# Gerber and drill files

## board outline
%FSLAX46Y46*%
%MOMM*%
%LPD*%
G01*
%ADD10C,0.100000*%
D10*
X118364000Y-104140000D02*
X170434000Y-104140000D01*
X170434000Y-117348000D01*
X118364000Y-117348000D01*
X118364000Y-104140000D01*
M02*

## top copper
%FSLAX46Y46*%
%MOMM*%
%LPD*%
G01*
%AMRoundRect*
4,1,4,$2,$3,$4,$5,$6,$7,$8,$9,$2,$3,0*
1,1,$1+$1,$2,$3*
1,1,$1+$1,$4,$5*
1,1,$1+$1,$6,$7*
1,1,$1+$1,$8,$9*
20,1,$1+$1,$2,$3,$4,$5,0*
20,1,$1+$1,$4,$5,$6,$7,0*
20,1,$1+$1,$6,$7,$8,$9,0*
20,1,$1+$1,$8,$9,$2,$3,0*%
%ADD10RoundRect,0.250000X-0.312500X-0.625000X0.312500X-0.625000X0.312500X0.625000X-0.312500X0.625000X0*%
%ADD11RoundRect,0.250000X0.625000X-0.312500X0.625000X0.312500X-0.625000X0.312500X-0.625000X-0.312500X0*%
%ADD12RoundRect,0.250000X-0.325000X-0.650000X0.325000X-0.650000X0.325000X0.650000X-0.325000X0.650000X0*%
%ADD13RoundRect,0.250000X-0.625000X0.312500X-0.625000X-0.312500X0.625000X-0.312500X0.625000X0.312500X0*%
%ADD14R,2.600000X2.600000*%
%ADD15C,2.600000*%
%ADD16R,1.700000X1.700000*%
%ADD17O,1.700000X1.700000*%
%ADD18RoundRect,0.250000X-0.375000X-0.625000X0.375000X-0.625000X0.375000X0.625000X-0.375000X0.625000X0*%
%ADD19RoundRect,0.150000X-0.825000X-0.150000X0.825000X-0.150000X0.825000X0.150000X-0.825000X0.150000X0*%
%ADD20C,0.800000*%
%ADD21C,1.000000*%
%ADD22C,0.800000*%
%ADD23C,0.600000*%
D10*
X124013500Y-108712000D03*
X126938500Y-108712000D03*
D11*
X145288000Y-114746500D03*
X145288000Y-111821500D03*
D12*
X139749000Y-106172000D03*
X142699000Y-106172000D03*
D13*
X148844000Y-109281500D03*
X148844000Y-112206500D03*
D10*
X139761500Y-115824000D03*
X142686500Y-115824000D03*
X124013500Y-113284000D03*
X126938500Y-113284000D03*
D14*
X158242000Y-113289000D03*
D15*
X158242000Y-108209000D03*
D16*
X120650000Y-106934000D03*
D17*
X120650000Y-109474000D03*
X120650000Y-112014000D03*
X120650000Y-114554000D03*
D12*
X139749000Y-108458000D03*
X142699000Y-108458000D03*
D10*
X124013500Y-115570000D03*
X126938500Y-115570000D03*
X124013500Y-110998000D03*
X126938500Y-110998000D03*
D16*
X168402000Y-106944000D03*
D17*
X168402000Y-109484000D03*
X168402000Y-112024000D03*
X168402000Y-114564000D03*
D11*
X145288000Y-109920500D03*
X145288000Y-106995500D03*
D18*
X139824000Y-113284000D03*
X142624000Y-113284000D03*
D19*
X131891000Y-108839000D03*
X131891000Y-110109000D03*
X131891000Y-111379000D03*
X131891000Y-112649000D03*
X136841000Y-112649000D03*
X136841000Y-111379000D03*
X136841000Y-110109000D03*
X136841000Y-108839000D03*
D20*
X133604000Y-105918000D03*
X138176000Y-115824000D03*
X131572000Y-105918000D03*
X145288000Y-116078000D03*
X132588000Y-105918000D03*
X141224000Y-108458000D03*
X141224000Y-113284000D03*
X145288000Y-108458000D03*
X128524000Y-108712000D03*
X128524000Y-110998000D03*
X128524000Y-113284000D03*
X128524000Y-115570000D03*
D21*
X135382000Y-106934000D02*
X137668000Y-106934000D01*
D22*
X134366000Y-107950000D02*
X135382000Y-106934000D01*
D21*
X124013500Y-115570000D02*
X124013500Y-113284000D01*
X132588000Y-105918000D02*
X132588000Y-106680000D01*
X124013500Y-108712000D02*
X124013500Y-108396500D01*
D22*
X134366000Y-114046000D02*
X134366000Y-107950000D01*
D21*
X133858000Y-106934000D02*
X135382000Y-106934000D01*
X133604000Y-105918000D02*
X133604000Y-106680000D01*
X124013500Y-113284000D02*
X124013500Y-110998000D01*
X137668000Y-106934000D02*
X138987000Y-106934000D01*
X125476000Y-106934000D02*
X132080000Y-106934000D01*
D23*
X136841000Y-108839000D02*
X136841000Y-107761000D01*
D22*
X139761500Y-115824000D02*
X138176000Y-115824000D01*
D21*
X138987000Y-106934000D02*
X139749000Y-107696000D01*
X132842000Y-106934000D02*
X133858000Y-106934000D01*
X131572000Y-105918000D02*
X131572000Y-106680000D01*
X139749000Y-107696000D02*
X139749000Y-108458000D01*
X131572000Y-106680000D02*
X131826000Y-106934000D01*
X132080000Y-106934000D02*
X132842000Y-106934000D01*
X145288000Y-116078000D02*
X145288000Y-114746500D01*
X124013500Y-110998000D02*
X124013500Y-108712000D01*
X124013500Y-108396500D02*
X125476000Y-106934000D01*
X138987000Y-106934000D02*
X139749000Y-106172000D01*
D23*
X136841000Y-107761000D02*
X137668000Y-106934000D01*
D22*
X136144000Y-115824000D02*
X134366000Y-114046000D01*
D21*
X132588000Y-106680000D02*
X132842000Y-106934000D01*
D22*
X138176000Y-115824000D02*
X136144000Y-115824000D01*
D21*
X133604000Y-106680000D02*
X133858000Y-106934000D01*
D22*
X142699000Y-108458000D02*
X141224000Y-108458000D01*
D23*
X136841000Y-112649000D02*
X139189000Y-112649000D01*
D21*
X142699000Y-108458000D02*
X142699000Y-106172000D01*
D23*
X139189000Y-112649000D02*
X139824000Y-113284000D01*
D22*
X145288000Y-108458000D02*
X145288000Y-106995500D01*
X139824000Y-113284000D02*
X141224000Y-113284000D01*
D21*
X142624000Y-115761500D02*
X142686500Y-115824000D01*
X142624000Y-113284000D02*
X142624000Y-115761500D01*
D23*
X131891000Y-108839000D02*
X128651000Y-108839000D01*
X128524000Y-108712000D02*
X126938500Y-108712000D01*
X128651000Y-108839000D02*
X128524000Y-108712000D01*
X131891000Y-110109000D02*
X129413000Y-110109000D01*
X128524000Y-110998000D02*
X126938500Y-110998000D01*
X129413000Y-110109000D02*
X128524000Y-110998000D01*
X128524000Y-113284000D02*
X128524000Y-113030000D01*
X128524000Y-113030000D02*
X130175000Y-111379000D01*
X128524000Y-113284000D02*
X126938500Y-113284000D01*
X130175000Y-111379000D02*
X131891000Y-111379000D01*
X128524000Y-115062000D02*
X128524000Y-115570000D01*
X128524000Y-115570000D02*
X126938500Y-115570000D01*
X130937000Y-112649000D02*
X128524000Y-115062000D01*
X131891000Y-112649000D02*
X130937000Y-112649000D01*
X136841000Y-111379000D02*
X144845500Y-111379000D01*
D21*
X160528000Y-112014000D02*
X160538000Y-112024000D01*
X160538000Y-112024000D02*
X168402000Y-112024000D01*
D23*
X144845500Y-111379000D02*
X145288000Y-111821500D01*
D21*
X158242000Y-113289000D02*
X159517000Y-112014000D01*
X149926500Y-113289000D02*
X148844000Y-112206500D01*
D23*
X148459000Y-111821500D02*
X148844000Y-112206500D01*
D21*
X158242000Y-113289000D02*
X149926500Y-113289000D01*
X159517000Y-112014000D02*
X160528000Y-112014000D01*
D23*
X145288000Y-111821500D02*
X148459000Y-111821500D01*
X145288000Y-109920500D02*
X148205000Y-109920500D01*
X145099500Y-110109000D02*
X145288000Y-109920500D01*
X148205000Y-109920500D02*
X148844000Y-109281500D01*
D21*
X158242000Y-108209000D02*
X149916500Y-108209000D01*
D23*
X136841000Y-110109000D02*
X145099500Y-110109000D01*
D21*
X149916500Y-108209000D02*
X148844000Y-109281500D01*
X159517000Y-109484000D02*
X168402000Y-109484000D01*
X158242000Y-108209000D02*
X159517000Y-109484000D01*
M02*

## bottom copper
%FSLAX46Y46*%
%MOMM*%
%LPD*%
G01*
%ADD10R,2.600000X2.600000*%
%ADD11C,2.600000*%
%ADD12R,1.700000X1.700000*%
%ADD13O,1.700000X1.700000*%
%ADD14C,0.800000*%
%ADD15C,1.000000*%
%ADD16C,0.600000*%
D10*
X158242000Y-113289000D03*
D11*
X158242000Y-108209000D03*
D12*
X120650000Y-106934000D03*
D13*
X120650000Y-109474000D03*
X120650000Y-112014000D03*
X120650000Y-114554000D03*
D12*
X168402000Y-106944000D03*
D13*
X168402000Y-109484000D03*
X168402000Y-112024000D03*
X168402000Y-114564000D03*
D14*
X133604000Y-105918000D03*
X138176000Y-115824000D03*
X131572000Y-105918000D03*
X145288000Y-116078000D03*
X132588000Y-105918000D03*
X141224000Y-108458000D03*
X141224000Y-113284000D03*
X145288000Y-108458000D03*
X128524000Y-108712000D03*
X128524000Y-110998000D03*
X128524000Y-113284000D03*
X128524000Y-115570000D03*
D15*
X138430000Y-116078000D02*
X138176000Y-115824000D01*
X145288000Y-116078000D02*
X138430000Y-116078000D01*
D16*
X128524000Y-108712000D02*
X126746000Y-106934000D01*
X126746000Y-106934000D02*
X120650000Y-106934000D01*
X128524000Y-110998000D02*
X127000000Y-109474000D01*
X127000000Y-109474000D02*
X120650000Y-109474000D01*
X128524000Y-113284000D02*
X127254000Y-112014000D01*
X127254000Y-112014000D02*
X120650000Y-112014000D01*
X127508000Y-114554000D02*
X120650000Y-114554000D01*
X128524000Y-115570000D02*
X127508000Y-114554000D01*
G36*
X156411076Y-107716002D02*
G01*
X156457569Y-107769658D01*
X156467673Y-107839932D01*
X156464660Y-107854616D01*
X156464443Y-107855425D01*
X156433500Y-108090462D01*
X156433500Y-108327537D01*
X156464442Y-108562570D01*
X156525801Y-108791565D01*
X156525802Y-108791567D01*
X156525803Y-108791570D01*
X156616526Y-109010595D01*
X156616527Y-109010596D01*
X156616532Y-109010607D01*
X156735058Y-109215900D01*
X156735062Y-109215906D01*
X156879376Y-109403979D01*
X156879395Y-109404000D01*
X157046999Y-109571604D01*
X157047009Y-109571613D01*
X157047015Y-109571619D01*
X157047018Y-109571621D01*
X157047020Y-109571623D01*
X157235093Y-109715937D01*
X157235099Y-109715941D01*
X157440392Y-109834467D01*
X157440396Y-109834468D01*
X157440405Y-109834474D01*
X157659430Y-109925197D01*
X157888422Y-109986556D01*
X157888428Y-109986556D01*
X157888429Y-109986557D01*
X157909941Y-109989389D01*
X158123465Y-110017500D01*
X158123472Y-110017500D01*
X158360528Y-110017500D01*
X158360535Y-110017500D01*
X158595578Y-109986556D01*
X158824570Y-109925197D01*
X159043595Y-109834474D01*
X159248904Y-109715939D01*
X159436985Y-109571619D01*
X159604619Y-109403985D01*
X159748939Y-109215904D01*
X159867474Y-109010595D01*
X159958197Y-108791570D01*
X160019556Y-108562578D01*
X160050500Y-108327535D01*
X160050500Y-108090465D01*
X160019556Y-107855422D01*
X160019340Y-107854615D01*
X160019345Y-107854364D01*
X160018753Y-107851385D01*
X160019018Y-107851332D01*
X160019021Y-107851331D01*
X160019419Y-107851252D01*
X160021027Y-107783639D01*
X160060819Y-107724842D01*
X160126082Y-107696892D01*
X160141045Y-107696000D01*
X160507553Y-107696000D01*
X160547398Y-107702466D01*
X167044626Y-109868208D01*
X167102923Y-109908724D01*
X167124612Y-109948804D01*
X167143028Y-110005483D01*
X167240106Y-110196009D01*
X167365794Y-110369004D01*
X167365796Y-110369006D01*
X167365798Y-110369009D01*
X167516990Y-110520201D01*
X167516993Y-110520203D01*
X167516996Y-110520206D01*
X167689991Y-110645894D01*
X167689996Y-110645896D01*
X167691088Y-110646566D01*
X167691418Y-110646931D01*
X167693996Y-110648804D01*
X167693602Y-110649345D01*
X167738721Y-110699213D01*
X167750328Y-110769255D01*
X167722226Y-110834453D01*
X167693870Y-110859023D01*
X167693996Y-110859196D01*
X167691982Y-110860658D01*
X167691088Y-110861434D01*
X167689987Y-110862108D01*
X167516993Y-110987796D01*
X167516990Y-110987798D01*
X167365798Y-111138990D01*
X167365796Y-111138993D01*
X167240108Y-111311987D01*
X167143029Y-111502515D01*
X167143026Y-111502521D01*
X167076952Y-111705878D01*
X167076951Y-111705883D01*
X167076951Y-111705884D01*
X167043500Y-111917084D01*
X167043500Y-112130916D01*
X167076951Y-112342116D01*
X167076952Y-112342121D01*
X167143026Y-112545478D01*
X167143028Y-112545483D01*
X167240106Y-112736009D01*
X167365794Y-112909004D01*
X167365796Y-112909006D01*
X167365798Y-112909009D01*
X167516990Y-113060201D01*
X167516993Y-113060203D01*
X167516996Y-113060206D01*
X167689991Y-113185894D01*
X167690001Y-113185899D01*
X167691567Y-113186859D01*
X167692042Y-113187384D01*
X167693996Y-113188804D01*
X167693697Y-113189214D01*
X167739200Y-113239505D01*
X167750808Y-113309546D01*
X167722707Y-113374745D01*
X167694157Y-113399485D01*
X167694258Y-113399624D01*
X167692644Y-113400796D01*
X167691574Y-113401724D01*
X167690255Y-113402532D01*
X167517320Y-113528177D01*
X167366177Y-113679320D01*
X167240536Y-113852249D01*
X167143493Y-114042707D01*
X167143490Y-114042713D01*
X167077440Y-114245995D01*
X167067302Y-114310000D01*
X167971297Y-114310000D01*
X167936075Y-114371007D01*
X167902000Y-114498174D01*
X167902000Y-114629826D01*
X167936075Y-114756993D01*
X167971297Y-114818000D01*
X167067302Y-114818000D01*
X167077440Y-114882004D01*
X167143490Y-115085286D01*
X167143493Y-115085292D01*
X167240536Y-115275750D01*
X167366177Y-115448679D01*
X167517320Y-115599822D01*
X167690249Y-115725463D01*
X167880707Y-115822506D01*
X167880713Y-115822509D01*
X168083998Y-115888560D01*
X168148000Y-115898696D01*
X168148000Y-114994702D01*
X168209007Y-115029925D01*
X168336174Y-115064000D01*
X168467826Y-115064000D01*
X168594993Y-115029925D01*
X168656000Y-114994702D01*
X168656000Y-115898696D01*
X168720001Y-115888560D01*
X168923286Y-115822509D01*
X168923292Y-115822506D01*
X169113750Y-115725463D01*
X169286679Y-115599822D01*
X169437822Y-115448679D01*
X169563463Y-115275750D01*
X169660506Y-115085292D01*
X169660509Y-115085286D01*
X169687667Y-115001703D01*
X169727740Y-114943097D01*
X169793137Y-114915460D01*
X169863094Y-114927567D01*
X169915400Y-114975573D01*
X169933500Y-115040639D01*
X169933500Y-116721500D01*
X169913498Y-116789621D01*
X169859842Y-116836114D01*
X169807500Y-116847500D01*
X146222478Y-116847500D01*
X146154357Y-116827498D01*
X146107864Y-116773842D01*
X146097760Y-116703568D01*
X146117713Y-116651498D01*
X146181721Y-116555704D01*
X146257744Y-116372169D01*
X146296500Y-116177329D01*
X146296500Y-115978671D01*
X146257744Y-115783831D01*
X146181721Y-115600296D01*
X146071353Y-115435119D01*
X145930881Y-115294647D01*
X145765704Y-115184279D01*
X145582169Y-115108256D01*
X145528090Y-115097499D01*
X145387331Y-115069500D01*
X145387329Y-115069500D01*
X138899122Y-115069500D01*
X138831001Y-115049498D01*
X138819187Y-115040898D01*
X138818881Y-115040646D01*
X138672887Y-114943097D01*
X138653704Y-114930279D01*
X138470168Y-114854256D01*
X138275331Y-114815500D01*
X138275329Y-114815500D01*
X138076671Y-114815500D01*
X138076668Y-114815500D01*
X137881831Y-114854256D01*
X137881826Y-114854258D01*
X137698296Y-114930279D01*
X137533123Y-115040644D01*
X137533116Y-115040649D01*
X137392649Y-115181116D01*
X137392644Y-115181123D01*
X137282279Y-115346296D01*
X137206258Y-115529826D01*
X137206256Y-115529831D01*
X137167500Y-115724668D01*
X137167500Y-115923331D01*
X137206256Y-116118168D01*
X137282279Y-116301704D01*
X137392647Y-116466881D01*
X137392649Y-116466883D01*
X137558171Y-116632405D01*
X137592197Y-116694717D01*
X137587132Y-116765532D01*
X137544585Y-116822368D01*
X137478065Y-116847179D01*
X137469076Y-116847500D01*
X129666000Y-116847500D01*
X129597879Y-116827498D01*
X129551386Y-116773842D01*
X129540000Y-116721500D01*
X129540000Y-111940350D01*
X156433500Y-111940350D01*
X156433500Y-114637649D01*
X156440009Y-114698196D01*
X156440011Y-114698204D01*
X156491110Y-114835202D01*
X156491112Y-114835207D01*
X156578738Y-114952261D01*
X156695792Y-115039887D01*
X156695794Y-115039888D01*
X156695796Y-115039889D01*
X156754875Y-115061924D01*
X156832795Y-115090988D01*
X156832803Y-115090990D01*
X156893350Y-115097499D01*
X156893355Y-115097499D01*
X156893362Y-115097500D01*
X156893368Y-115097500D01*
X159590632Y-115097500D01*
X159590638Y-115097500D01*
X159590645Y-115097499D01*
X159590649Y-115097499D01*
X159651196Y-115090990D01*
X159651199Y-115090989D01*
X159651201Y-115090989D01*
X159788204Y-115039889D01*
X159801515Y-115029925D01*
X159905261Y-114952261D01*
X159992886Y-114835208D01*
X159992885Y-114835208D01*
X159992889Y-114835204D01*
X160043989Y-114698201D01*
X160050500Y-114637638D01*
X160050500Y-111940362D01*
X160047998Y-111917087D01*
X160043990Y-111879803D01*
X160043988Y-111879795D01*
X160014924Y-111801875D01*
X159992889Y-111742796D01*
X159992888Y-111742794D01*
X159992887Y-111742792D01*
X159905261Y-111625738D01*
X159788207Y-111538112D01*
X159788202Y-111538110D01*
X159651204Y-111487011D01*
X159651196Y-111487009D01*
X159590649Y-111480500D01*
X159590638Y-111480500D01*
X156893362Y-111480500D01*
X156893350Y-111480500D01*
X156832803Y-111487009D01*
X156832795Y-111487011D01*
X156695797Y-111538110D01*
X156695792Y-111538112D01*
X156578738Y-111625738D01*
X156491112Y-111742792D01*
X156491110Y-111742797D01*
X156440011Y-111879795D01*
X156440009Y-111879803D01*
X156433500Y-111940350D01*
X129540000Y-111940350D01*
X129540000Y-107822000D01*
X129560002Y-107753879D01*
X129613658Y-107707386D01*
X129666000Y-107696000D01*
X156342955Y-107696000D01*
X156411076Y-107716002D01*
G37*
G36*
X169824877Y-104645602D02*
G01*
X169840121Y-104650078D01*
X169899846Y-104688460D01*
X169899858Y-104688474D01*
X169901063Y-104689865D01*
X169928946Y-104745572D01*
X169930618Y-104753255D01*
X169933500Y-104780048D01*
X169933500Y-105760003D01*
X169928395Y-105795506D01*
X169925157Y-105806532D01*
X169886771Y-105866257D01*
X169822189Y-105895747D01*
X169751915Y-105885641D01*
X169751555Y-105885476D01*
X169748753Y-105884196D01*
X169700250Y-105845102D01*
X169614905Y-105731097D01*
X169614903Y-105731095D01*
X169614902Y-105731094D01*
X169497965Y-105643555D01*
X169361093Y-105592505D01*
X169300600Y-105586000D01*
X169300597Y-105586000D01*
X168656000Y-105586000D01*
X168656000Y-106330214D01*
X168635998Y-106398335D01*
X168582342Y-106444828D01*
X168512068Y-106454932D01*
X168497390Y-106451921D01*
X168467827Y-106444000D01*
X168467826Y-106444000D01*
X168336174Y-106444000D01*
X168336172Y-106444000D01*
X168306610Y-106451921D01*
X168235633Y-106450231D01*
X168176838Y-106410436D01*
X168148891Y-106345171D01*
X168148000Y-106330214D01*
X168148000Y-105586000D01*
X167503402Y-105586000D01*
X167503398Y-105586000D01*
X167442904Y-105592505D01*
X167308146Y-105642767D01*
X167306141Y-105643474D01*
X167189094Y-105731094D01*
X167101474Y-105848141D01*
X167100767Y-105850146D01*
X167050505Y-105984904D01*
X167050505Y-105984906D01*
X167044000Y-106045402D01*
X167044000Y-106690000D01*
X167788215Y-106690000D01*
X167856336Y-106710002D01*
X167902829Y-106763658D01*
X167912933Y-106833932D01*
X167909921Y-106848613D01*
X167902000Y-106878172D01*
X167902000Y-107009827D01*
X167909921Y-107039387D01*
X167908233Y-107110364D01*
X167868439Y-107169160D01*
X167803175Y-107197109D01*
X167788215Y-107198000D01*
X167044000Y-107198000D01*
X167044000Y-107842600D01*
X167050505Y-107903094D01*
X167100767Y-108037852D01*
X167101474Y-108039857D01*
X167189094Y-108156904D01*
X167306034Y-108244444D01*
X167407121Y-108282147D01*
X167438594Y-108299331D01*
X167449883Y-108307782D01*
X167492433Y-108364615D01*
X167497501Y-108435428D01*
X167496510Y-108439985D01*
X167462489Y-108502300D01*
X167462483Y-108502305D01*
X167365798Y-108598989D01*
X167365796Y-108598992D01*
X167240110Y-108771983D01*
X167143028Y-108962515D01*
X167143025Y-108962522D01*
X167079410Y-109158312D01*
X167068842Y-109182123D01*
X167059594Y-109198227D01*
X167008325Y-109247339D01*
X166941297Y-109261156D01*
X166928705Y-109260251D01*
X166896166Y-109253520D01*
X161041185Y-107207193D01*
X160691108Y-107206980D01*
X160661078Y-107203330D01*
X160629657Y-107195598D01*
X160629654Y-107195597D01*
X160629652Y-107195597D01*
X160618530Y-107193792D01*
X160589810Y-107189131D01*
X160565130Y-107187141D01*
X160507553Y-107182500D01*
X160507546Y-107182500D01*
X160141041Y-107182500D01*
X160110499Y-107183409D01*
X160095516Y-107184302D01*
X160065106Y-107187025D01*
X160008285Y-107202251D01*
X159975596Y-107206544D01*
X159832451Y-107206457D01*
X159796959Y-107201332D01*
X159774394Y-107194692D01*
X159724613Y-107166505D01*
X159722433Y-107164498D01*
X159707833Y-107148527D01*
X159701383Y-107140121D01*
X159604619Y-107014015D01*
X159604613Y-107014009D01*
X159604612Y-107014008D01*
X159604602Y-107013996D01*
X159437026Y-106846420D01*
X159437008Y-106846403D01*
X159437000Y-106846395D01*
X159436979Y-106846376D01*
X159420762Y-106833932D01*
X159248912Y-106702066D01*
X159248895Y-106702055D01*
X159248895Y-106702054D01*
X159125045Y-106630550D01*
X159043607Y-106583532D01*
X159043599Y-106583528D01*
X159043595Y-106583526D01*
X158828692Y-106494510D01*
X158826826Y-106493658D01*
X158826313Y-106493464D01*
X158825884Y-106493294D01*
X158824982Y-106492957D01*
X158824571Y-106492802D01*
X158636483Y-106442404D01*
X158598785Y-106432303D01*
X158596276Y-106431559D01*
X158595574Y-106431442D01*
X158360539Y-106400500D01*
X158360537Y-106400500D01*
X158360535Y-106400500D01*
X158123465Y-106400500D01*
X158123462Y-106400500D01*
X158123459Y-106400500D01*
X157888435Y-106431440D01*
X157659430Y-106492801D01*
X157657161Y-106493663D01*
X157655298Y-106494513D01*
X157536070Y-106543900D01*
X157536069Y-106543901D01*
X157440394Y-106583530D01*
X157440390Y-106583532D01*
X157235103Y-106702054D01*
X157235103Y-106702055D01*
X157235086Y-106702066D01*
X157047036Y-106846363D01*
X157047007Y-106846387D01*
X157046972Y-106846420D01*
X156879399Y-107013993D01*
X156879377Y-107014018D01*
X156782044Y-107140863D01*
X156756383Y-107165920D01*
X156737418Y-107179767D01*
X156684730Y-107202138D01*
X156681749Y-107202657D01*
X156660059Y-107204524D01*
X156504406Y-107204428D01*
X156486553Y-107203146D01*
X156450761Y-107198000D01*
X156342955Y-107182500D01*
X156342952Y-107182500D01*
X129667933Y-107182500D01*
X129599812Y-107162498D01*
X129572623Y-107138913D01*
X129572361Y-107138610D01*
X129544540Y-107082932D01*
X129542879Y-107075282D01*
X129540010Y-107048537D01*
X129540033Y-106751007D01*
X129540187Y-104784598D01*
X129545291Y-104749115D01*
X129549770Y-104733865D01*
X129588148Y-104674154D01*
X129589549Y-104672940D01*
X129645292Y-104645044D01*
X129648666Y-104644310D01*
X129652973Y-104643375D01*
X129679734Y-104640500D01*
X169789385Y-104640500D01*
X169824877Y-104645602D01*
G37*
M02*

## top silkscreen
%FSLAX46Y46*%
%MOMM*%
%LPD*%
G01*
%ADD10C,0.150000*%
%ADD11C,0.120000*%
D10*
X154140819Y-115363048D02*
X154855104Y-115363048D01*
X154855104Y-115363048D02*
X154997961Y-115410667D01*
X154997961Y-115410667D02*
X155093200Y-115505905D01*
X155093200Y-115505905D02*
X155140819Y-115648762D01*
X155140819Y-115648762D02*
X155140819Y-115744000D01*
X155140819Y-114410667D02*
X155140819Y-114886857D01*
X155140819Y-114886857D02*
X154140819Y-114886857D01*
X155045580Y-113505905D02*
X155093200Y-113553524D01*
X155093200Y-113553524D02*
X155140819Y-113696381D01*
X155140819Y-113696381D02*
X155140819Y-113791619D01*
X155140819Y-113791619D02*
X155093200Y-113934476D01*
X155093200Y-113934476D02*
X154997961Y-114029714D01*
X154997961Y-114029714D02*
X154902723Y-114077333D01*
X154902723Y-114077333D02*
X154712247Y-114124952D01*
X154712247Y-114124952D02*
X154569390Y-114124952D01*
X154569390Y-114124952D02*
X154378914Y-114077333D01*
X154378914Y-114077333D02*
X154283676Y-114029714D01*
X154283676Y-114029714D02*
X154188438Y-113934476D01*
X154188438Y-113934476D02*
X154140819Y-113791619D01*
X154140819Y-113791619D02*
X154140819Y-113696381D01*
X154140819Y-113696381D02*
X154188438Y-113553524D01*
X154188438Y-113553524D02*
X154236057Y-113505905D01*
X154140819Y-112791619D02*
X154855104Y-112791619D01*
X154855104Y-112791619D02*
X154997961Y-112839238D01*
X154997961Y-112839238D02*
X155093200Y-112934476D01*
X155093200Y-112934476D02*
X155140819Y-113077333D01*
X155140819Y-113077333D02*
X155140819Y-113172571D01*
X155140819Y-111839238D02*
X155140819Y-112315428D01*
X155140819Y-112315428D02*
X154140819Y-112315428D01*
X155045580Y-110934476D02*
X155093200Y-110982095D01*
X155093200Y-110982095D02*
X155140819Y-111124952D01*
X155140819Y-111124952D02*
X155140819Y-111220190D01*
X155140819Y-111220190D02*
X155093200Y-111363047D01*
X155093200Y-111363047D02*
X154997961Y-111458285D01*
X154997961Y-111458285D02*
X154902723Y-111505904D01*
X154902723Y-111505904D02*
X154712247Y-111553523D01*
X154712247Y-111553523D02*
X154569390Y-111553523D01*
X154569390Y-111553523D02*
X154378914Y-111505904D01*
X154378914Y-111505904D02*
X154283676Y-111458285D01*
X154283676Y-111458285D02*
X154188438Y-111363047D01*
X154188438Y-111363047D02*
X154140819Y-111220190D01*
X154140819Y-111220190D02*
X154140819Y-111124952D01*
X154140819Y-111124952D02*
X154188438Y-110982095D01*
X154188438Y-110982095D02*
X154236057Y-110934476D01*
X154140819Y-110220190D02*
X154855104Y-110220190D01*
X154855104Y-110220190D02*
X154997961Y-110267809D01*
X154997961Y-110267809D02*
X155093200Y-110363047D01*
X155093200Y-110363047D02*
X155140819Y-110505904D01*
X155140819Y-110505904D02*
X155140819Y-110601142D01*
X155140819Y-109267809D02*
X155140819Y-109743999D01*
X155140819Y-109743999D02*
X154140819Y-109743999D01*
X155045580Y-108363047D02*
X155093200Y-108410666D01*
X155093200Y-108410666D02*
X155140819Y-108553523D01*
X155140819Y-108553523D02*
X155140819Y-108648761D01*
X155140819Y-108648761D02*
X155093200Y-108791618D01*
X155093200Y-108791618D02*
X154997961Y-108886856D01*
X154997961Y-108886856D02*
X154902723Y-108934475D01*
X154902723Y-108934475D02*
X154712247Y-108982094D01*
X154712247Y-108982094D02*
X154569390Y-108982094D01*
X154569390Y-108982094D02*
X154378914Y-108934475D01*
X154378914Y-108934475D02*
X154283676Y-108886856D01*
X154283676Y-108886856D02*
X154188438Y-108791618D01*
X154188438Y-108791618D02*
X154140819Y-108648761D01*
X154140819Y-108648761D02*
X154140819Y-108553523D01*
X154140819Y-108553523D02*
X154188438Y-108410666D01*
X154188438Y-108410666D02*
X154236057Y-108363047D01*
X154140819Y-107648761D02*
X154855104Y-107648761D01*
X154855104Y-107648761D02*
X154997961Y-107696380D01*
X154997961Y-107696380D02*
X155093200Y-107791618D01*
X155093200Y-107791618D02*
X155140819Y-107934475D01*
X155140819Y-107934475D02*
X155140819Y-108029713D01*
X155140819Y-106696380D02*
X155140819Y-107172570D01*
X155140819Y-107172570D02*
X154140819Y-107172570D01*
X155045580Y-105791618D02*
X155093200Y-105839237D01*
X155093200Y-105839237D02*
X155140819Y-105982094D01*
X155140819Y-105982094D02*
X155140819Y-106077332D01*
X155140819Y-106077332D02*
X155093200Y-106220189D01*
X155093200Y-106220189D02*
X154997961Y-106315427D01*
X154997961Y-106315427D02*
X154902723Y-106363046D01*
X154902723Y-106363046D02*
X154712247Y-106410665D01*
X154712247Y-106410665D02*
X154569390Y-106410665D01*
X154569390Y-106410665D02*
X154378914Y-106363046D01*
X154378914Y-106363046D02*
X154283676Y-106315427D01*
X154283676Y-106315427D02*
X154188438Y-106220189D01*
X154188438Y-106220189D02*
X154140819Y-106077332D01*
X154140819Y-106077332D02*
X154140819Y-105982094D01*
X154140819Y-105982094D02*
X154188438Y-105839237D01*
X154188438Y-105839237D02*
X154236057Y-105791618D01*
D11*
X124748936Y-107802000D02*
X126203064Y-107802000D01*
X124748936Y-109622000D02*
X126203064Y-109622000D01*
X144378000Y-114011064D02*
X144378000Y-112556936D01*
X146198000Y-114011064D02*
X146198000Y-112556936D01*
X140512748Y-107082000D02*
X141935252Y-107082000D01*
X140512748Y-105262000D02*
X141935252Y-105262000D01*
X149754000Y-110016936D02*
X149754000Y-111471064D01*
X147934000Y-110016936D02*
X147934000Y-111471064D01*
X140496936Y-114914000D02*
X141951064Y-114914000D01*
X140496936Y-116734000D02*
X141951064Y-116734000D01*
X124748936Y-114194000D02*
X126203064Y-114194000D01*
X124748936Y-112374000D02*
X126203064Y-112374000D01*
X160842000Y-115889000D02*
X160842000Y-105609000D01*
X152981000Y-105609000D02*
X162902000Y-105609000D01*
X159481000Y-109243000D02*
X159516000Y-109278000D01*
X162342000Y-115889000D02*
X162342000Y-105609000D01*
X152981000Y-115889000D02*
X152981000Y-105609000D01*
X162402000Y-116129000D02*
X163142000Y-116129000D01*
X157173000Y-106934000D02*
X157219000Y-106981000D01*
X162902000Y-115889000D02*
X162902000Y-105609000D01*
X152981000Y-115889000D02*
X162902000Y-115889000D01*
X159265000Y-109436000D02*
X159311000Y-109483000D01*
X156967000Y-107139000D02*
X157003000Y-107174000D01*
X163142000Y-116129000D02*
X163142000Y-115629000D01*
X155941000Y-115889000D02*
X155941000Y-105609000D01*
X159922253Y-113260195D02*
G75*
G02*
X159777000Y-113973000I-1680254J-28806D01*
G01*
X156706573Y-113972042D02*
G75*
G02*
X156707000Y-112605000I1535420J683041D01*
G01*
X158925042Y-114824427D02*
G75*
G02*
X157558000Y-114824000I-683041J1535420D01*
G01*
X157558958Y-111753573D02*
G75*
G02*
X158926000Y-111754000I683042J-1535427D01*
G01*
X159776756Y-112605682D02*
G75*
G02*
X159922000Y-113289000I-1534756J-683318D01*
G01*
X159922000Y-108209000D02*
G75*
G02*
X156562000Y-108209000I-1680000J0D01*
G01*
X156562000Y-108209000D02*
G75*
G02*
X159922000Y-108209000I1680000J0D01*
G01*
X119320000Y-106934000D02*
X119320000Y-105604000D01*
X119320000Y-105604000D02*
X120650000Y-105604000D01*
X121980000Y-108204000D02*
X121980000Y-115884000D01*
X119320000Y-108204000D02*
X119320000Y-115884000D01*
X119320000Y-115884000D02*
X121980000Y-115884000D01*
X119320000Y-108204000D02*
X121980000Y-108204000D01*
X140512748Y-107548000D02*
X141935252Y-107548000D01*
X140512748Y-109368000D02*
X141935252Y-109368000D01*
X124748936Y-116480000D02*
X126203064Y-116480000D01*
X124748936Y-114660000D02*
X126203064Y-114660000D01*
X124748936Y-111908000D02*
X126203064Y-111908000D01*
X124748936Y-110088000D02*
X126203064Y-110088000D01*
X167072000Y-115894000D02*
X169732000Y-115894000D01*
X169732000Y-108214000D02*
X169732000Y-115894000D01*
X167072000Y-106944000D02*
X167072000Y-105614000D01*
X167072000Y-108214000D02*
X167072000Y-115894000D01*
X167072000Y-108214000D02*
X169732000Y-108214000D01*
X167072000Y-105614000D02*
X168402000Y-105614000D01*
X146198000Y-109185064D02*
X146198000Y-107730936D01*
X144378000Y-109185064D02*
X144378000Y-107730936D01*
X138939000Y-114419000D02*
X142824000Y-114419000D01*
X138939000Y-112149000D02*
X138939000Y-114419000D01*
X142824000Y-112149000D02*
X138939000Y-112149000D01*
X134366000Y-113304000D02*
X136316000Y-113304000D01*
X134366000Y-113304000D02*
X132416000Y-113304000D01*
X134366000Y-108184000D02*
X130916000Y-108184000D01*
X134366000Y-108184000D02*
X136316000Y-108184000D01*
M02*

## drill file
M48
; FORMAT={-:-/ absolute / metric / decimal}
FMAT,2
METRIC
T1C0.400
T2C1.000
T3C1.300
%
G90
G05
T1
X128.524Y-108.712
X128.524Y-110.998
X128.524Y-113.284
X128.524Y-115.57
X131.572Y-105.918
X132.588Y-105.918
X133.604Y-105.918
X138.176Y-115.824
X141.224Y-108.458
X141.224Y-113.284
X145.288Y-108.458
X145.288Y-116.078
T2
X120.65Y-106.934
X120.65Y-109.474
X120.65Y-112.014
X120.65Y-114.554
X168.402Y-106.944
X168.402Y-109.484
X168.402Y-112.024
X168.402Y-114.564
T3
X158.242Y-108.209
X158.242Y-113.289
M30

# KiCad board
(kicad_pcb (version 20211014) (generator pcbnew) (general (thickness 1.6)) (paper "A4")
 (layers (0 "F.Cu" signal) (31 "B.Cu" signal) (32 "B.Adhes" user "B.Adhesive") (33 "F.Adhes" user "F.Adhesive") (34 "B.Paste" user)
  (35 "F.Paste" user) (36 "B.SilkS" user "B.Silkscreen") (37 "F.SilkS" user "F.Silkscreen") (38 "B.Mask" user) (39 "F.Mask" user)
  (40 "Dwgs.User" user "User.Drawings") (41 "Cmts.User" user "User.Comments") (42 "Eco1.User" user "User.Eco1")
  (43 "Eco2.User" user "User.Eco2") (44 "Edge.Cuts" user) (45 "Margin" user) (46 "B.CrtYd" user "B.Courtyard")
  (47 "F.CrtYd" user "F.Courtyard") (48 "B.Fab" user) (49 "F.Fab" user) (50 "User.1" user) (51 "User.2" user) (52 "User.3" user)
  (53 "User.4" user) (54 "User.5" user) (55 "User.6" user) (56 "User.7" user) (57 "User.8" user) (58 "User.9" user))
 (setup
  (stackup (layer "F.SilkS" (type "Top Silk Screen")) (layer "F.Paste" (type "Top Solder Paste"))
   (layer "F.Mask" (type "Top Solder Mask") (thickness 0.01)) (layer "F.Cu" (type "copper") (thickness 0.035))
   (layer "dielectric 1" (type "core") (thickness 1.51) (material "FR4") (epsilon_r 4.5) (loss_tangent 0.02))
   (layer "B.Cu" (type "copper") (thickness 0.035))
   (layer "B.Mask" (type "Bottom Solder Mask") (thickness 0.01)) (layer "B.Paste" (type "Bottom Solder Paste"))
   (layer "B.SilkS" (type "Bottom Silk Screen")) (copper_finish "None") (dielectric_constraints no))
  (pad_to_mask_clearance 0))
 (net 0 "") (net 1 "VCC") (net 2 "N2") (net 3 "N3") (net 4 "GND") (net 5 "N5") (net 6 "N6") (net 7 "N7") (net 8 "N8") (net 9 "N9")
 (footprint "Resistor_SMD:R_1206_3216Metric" (layer "F.Cu") (at 125.476 108.712)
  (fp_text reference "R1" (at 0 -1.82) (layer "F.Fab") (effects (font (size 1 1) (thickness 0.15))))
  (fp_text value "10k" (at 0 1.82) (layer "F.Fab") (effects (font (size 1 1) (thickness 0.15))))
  (fp_line (start -0.727064 -0.91) (end 0.727064 -0.91) (layer "F.SilkS") (width 0.12))
  (fp_line (start -0.727064 0.91) (end 0.727064 0.91) (layer "F.SilkS") (width 0.12))
  (pad "1" smd roundrect locked (at -1.4625 0) (size 1.125 1.75) (layers "F.Cu" "F.Paste" "F.Mask") (roundrect_rratio 0.222222)
   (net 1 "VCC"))
  (pad "2" smd roundrect locked (at 1.4625 0) (size 1.125 1.75) (layers "F.Cu" "F.Paste" "F.Mask") (roundrect_rratio 0.222222) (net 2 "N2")))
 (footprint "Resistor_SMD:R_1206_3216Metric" (layer "F.Cu") (at 145.288 113.284 90)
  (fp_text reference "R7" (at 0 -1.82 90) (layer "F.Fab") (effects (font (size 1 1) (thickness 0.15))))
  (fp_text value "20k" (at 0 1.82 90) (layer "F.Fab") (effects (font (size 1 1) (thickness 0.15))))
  (fp_line (start -0.727064 -0.91) (end 0.727064 -0.91) (layer "F.SilkS") (width 0.12))
  (fp_line (start -0.727064 0.91) (end 0.727064 0.91) (layer "F.SilkS") (width 0.12))
  (pad "1" smd roundrect locked (at -1.4625 0 90) (size 1.125 1.75) (layers "F.Cu" "F.Paste" "F.Mask") (roundrect_rratio 0.222222)
   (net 1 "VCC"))
  (pad "2" smd roundrect locked (at 1.4625 0 90) (size 1.125 1.75) (layers "F.Cu" "F.Paste" "F.Mask") (roundrect_rratio 0.222222)
   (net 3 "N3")))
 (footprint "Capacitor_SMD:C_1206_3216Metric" (layer "F.Cu") (at 141.224 106.172)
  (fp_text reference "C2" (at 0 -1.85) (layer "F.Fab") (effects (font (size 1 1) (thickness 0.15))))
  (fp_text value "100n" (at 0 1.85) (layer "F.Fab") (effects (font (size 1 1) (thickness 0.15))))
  (fp_line (start -0.711252 0.91) (end 0.711252 0.91) (layer "F.SilkS") (width 0.12))
  (fp_line (start -0.711252 -0.91) (end 0.711252 -0.91) (layer "F.SilkS") (width 0.12))
  (pad "1" smd roundrect locked (at -1.475 0) (size 1.15 1.8) (layers "F.Cu" "F.Paste" "F.Mask") (roundrect_rratio 0.217391) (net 1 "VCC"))
  (pad "2" smd roundrect locked (at 1.475 0) (size 1.15 1.8) (layers "F.Cu" "F.Paste" "F.Mask") (roundrect_rratio 0.217391) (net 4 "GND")))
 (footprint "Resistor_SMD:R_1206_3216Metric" (layer "F.Cu") (at 148.844 110.744 -90)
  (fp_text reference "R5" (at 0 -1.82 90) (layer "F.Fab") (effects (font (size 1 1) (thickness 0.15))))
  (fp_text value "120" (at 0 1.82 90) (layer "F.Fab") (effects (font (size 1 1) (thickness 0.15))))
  (fp_line (start -0.727064 -0.91) (end 0.727064 -0.91) (layer "F.SilkS") (width 0.12))
  (fp_line (start -0.727064 0.91) (end 0.727064 0.91) (layer "F.SilkS") (width 0.12))
  (pad "1" smd roundrect locked (at -1.4625 0 270) (size 1.125 1.75) (layers "F.Cu" "F.Paste" "F.Mask") (roundrect_rratio 0.222222)
   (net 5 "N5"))
  (pad "2" smd roundrect locked (at 1.4625 0 270) (size 1.125 1.75) (layers "F.Cu" "F.Paste" "F.Mask") (roundrect_rratio 0.222222)
   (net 3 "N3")))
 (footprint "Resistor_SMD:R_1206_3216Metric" (layer "F.Cu") (at 141.224 115.824)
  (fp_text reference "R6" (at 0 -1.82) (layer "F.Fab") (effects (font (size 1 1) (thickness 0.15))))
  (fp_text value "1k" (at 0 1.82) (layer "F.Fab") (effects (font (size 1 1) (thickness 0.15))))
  (fp_line (start -0.727064 -0.91) (end 0.727064 -0.91) (layer "F.SilkS") (width 0.12))
  (fp_line (start -0.727064 0.91) (end 0.727064 0.91) (layer "F.SilkS") (width 0.12))
  (pad "1" smd roundrect locked (at -1.4625 0) (size 1.125 1.75) (layers "F.Cu" "F.Paste" "F.Mask") (roundrect_rratio 0.222222)
   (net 1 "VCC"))
  (pad "2" smd roundrect locked (at 1.4625 0) (size 1.125 1.75) (layers "F.Cu" "F.Paste" "F.Mask") (roundrect_rratio 0.222222) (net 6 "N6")))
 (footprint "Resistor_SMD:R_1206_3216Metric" (layer "F.Cu") (at 125.476 113.284)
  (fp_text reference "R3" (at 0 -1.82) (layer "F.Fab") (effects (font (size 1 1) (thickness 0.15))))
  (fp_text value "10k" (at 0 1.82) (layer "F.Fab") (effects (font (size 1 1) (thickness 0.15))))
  (fp_line (start -0.727064 0.91) (end 0.727064 0.91) (layer "F.SilkS") (width 0.12))
  (fp_line (start -0.727064 -0.91) (end 0.727064 -0.91) (layer "F.SilkS") (width 0.12))
  (pad "1" smd roundrect locked (at -1.4625 0) (size 1.125 1.75) (layers "F.Cu" "F.Paste" "F.Mask") (roundrect_rratio 0.222222)
   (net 1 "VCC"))
  (pad "2" smd roundrect locked (at 1.4625 0) (size 1.125 1.75) (layers "F.Cu" "F.Paste" "F.Mask") (roundrect_rratio 0.222222) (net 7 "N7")))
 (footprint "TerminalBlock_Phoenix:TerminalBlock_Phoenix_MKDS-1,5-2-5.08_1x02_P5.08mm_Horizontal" (layer "F.Cu") (at 158.242 113.289 90)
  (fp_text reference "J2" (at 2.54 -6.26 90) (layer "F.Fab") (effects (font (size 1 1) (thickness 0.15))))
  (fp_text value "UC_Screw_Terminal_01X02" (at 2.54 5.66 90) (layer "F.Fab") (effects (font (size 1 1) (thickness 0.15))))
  (fp_line (start -2.6 2.6) (end 7.68 2.6) (layer "F.SilkS") (width 0.12))
  (fp_line (start 7.68 -5.261) (end 7.68 4.66) (layer "F.SilkS") (width 0.12))
  (fp_line (start 4.046 1.239) (end 4.011 1.274) (layer "F.SilkS") (width 0.12))
  (fp_line (start -2.6 4.1) (end 7.68 4.1) (layer "F.SilkS") (width 0.12))
  (fp_line (start -2.6 -5.261) (end 7.68 -5.261) (layer "F.SilkS") (width 0.12))
  (fp_line (start -2.84 4.16) (end -2.84 4.9) (layer "F.SilkS") (width 0.12))
  (fp_line (start 6.355 -1.069) (end 6.308 -1.023) (layer "F.SilkS") (width 0.12))
  (fp_line (start -2.6 4.66) (end 7.68 4.66) (layer "F.SilkS") (width 0.12))
  (fp_line (start -2.6 -5.261) (end -2.6 4.66) (layer "F.SilkS") (width 0.12))
  (fp_line (start 3.853 1.023) (end 3.806 1.069) (layer "F.SilkS") (width 0.12))
  (fp_line (start 6.15 -1.275) (end 6.115 -1.239) (layer "F.SilkS") (width 0.12))
  (fp_line (start -2.84 4.9) (end -2.34 4.9) (layer "F.SilkS") (width 0.12))
  (fp_line (start -2.6 -2.301) (end 7.68 -2.301) (layer "F.SilkS") (width 0.12))
  (fp_arc (start 0.028805 1.680253) (mid -0.335551 1.646659) (end -0.684 1.535) (layer "F.SilkS") (width 0.12))
  (fp_arc (start -0.683042 -1.535427) (mid 0.000524 -1.680501) (end 0.684 -1.535) (layer "F.SilkS") (width 0.12))
  (fp_arc (start -1.535427 0.683042) (mid -1.680501 -0.000524) (end -1.535 -0.684) (layer "F.SilkS") (width 0.12))
  (fp_arc (start 1.535427 -0.683042) (mid 1.680501 0.000524) (end 1.535 0.684) (layer "F.SilkS") (width 0.12))
  (fp_arc (start 0.683318 1.534756) (mid 0.349292 1.643288) (end 0 1.68) (layer "F.SilkS") (width 0.12))
  (fp_circle (center 5.08 0) (end 6.76 0) (layer "F.SilkS") (width 0.12) (fill none))
  (pad "1" thru_hole rect locked (at 0 0 90) (size 2.6 2.6) (drill 1.3) (layers *.Cu *.Mask) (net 3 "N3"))
  (pad "2" thru_hole circle locked (at 5.08 0 90) (size 2.6 2.6) (drill 1.3) (layers *.Cu *.Mask) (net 5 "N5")))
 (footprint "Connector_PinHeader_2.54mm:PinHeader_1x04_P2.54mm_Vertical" (layer "F.Cu") (at 120.65 106.934)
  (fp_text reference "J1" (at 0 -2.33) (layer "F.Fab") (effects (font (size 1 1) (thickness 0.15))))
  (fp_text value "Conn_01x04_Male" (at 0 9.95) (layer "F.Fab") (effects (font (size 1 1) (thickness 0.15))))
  (fp_line (start -1.33 0) (end -1.33 -1.33) (layer "F.SilkS") (width 0.12))
  (fp_line (start -1.33 -1.33) (end 0 -1.33) (layer "F.SilkS") (width 0.12))
  (fp_line (start 1.33 1.27) (end 1.33 8.95) (layer "F.SilkS") (width 0.12))
  (fp_line (start -1.33 1.27) (end -1.33 8.95) (layer "F.SilkS") (width 0.12))
  (fp_line (start -1.33 8.95) (end 1.33 8.95) (layer "F.SilkS") (width 0.12))
  (fp_line (start -1.33 1.27) (end 1.33 1.27) (layer "F.SilkS") (width 0.12))
  (pad "1" thru_hole rect locked (at 0 0) (size 1.7 1.7) (drill 1) (layers *.Cu *.Mask) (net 2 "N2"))
  (pad "2" thru_hole oval locked (at 0 2.54) (size 1.7 1.7) (drill 1) (layers *.Cu *.Mask) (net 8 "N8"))
  (pad "3" thru_hole oval locked (at 0 5.08) (size 1.7 1.7) (drill 1) (layers *.Cu *.Mask) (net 7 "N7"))
  (pad "4" thru_hole oval locked (at 0 7.62) (size 1.7 1.7) (drill 1) (layers *.Cu *.Mask) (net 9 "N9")))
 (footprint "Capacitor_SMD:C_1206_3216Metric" (layer "F.Cu") (at 141.224 108.458)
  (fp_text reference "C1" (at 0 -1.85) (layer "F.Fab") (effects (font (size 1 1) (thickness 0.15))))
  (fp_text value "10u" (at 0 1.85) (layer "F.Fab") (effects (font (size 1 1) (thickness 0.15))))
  (fp_line (start -0.711252 -0.91) (end 0.711252 -0.91) (layer "F.SilkS") (width 0.12))
  (fp_line (start -0.711252 0.91) (end 0.711252 0.91) (layer "F.SilkS") (width 0.12))
  (pad "1" smd roundrect locked (at -1.475 0) (size 1.15 1.8) (layers "F.Cu" "F.Paste" "F.Mask") (roundrect_rratio 0.217391) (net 1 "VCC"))
  (pad "2" smd roundrect locked (at 1.475 0) (size 1.15 1.8) (layers "F.Cu" "F.Paste" "F.Mask") (roundrect_rratio 0.217391) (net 4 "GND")))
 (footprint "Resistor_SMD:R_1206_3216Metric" (layer "F.Cu") (at 125.476 115.57)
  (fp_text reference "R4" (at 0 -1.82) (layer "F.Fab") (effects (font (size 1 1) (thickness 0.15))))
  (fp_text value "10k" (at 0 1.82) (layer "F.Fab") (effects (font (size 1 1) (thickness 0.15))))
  (fp_line (start -0.727064 0.91) (end 0.727064 0.91) (layer "F.SilkS") (width 0.12))
  (fp_line (start -0.727064 -0.91) (end 0.727064 -0.91) (layer "F.SilkS") (width 0.12))
  (pad "1" smd roundrect locked (at -1.4625 0) (size 1.125 1.75) (layers "F.Cu" "F.Paste" "F.Mask") (roundrect_rratio 0.222222)
   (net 1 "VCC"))
  (pad "2" smd roundrect locked (at 1.4625 0) (size 1.125 1.75) (layers "F.Cu" "F.Paste" "F.Mask") (roundrect_rratio 0.222222) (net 9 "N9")))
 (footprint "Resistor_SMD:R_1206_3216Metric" (layer "F.Cu") (at 125.476 110.998)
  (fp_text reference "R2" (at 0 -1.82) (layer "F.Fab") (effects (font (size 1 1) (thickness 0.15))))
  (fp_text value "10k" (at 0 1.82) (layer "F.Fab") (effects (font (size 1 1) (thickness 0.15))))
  (fp_line (start -0.727064 0.91) (end 0.727064 0.91) (layer "F.SilkS") (width 0.12))
  (fp_line (start -0.727064 -0.91) (end 0.727064 -0.91) (layer "F.SilkS") (width 0.12))
  (pad "1" smd roundrect locked (at -1.4625 0) (size 1.125 1.75) (layers "F.Cu" "F.Paste" "F.Mask") (roundrect_rratio 0.222222)
   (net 1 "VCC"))
  (pad "2" smd roundrect locked (at 1.4625 0) (size 1.125 1.75) (layers "F.Cu" "F.Paste" "F.Mask") (roundrect_rratio 0.222222) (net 8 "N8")))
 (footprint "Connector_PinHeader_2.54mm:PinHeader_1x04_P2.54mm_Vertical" (layer "F.Cu") (at 168.402 106.944)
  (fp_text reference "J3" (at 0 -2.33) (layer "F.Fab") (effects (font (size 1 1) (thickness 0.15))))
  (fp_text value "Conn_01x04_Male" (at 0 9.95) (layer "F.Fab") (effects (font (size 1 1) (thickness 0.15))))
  (fp_line (start -1.33 8.95) (end 1.33 8.95) (layer "F.SilkS") (width 0.12))
  (fp_line (start 1.33 1.27) (end 1.33 8.95) (layer "F.SilkS") (width 0.12))
  (fp_line (start -1.33 0) (end -1.33 -1.33) (layer "F.SilkS") (width 0.12))
  (fp_line (start -1.33 1.27) (end -1.33 8.95) (layer "F.SilkS") (width 0.12))
  (fp_line (start -1.33 1.27) (end 1.33 1.27) (layer "F.SilkS") (width 0.12))
  (fp_line (start -1.33 -1.33) (end 0 -1.33) (layer "F.SilkS") (width 0.12))
  (pad "1" thru_hole rect locked (at 0 0) (size 1.7 1.7) (drill 1) (layers *.Cu *.Mask) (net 1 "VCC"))
  (pad "2" thru_hole oval locked (at 0 2.54) (size 1.7 1.7) (drill 1) (layers *.Cu *.Mask) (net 5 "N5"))
  (pad "3" thru_hole oval locked (at 0 5.08) (size 1.7 1.7) (drill 1) (layers *.Cu *.Mask) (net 3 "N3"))
  (pad "4" thru_hole oval locked (at 0 7.62) (size 1.7 1.7) (drill 1) (layers *.Cu *.Mask) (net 4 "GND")))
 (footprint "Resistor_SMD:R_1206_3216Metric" (layer "F.Cu") (at 145.288 108.458 90)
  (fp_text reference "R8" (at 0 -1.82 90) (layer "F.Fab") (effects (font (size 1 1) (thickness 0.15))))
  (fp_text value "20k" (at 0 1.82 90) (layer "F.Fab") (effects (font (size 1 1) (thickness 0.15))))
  (fp_line (start -0.727064 0.91) (end 0.727064 0.91) (layer "F.SilkS") (width 0.12))
  (fp_line (start -0.727064 -0.91) (end 0.727064 -0.91) (layer "F.SilkS") (width 0.12))
  (pad "1" smd roundrect locked (at -1.4625 0 90) (size 1.125 1.75) (layers "F.Cu" "F.Paste" "F.Mask") (roundrect_rratio 0.222222)
   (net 5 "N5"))
  (pad "2" smd roundrect locked (at 1.4625 0 90) (size 1.125 1.75) (layers "F.Cu" "F.Paste" "F.Mask") (roundrect_rratio 0.222222)
   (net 4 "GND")))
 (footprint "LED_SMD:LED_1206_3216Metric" (layer "F.Cu") (at 141.224 113.284)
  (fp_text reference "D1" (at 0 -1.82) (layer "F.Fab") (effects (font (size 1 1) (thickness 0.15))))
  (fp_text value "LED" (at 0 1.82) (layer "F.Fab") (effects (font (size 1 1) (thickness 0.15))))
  (fp_line (start -2.285 1.135) (end 1.6 1.135) (layer "F.SilkS") (width 0.12))
  (fp_line (start -2.285 -1.135) (end -2.285 1.135) (layer "F.SilkS") (width 0.12))
  (fp_line (start 1.6 -1.135) (end -2.285 -1.135) (layer "F.SilkS") (width 0.12))
  (pad "1" smd roundrect locked (at -1.4 0) (size 1.25 1.75) (layers "F.Cu" "F.Paste" "F.Mask") (roundrect_rratio 0.2) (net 4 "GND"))
  (pad "2" smd roundrect locked (at 1.4 0) (size 1.25 1.75) (layers "F.Cu" "F.Paste" "F.Mask") (roundrect_rratio 0.2) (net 6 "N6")))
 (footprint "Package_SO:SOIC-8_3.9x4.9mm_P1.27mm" (layer "F.Cu") (at 134.366 110.744)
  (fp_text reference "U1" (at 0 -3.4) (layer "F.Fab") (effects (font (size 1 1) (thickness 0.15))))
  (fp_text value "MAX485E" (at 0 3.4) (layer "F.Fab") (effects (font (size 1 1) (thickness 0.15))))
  (fp_line (start 0 2.56) (end 1.95 2.56) (layer "F.SilkS") (width 0.12))
  (fp_line (start 0 2.56) (end -1.95 2.56) (layer "F.SilkS") (width 0.12))
  (fp_line (start 0 -2.56) (end -3.45 -2.56) (layer "F.SilkS") (width 0.12))
  (fp_line (start 0 -2.56) (end 1.95 -2.56) (layer "F.SilkS") (width 0.12))
  (pad "1" smd roundrect locked (at -2.475 -1.905) (size 1.95 0.6) (layers "F.Cu" "F.Paste" "F.Mask") (roundrect_rratio 0.25) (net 2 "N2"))
  (pad "2" smd roundrect locked (at -2.475 -0.635) (size 1.95 0.6) (layers "F.Cu" "F.Paste" "F.Mask") (roundrect_rratio 0.25) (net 8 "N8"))
  (pad "3" smd roundrect locked (at -2.475 0.635) (size 1.95 0.6) (layers "F.Cu" "F.Paste" "F.Mask") (roundrect_rratio 0.25) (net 7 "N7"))
  (pad "4" smd roundrect locked (at -2.475 1.905) (size 1.95 0.6) (layers "F.Cu" "F.Paste" "F.Mask") (roundrect_rratio 0.25) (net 9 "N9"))
  (pad "5" smd roundrect locked (at 2.475 1.905) (size 1.95 0.6) (layers "F.Cu" "F.Paste" "F.Mask") (roundrect_rratio 0.25) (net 4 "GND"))
  (pad "6" smd roundrect locked (at 2.475 0.635) (size 1.95 0.6) (layers "F.Cu" "F.Paste" "F.Mask") (roundrect_rratio 0.25) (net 3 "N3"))
  (pad "7" smd roundrect locked (at 2.475 -0.635) (size 1.95 0.6) (layers "F.Cu" "F.Paste" "F.Mask") (roundrect_rratio 0.25) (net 5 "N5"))
  (pad "8" smd roundrect locked (at 2.475 -1.905) (size 1.95 0.6) (layers "F.Cu" "F.Paste" "F.Mask") (roundrect_rratio 0.25) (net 1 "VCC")))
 (gr_rect (start 170.434 104.14) (end 118.364 117.348) (layer "Edge.Cuts") (width 0.1) (fill none))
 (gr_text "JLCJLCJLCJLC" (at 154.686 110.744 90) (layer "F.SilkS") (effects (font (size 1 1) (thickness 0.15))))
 (segment (start 135.382 106.934) (end 137.668 106.934) (width 1) (layer "F.Cu") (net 1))
 (segment (start 134.366 107.95) (end 135.382 106.934) (width 0.8) (layer "F.Cu") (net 1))
 (segment (start 124.0135 115.57) (end 124.0135 113.284) (width 1) (layer "F.Cu") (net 1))
 (segment (start 132.588 105.918) (end 132.588 106.68) (width 1) (layer "F.Cu") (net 1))
 (segment (start 124.0135 108.712) (end 124.0135 108.3965) (width 1) (layer "F.Cu") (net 1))
 (segment (start 134.366 114.046) (end 134.366 107.95) (width 0.8) (layer "F.Cu") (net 1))
 (segment (start 133.858 106.934) (end 135.382 106.934) (width 1) (layer "F.Cu") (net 1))
 (segment (start 133.604 105.918) (end 133.604 106.68) (width 1) (layer "F.Cu") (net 1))
 (segment (start 124.0135 113.284) (end 124.0135 110.998) (width 1) (layer "F.Cu") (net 1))
 (segment (start 137.668 106.934) (end 138.987 106.934) (width 1) (layer "F.Cu") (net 1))
 (segment (start 125.476 106.934) (end 132.08 106.934) (width 1) (layer "F.Cu") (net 1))
 (segment (start 136.841 108.839) (end 136.841 107.761) (width 0.6) (layer "F.Cu") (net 1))
 (segment (start 139.7615 115.824) (end 138.176 115.824) (width 0.8) (layer "F.Cu") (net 1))
 (segment (start 138.987 106.934) (end 139.749 107.696) (width 1) (layer "F.Cu") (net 1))
 (segment (start 132.842 106.934) (end 133.858 106.934) (width 1) (layer "F.Cu") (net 1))
 (segment (start 131.572 105.918) (end 131.572 106.68) (width 1) (layer "F.Cu") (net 1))
 (segment (start 139.749 107.696) (end 139.749 108.458) (width 1) (layer "F.Cu") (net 1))
 (segment (start 131.572 106.68) (end 131.826 106.934) (width 1) (layer "F.Cu") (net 1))
 (segment (start 132.08 106.934) (end 132.842 106.934) (width 1) (layer "F.Cu") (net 1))
 (segment (start 145.288 116.078) (end 145.288 114.7465) (width 1) (layer "F.Cu") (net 1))
 (segment (start 124.0135 110.998) (end 124.0135 108.712) (width 1) (layer "F.Cu") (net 1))
 (segment (start 124.0135 108.3965) (end 125.476 106.934) (width 1) (layer "F.Cu") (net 1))
 (segment (start 138.987 106.934) (end 139.749 106.172) (width 1) (layer "F.Cu") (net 1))
 (segment (start 136.841 107.761) (end 137.668 106.934) (width 0.6) (layer "F.Cu") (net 1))
 (segment (start 136.144 115.824) (end 134.366 114.046) (width 0.8) (layer "F.Cu") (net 1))
 (segment (start 132.588 106.68) (end 132.842 106.934) (width 1) (layer "F.Cu") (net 1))
 (segment (start 138.176 115.824) (end 136.144 115.824) (width 0.8) (layer "F.Cu") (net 1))
 (segment (start 133.604 106.68) (end 133.858 106.934) (width 1) (layer "F.Cu") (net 1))
 (via (at 133.604 105.918) (size 0.8) (drill 0.4) (layers "F.Cu" "B.Cu") (free) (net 1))
 (via (at 138.176 115.824) (size 0.8) (drill 0.4) (layers "F.Cu" "B.Cu") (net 1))
 (via (at 131.572 105.918) (size 0.8) (drill 0.4) (layers "F.Cu" "B.Cu") (free) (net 1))
 (via (at 145.288 116.078) (size 0.8) (drill 0.4) (layers "F.Cu" "B.Cu") (free) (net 1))
 (via (at 132.588 105.918) (size 0.8) (drill 0.4) (layers "F.Cu" "B.Cu") (free) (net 1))
 (segment (start 138.43 116.078) (end 138.176 115.824) (width 1) (layer "B.Cu") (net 1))
 (segment (start 145.288 116.078) (end 138.43 116.078) (width 1) (layer "B.Cu") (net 1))
 (segment (start 142.699 108.458) (end 141.224 108.458) (width 0.8) (layer "F.Cu") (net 4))
 (segment (start 136.841 112.649) (end 139.189 112.649) (width 0.6) (layer "F.Cu") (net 4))
 (segment (start 142.699 108.458) (end 142.699 106.172) (width 1) (layer "F.Cu") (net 4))
 (segment (start 139.189 112.649) (end 139.824 113.284) (width 0.6) (layer "F.Cu") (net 4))
 (segment (start 145.288 108.458) (end 145.288 106.9955) (width 0.8) (layer "F.Cu") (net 4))
 (segment (start 139.824 113.284) (end 141.224 113.284) (width 0.8) (layer "F.Cu") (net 4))
 (via (at 141.224 108.458) (size 0.8) (drill 0.4) (layers "F.Cu" "B.Cu") (free) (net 4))
 (via (at 141.224 113.284) (size 0.8) (drill 0.4) (layers "F.Cu" "B.Cu") (free) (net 4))
 (via (at 145.288 108.458) (size 0.8) (drill 0.4) (layers "F.Cu" "B.Cu") (free) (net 4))
 (segment (start 142.624 115.7615) (end 142.6865 115.824) (width 1) (layer "F.Cu") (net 6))
 (segment (start 142.624 113.284) (end 142.624 115.7615) (width 1) (layer "F.Cu") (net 6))
 (segment (start 131.891 108.839) (end 128.651 108.839) (width 0.6) (layer "F.Cu") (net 2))
 (segment (start 128.524 108.712) (end 126.9385 108.712) (width 0.6) (layer "F.Cu") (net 2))
 (segment (start 128.651 108.839) (end 128.524 108.712) (width 0.6) (layer "F.Cu") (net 2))
 (via (at 128.524 108.712) (size 0.8) (drill 0.4) (layers "F.Cu" "B.Cu") (free) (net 2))
 (segment (start 128.524 108.712) (end 126.746 106.934) (width 0.6) (layer "B.Cu") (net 2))
 (segment (start 126.746 106.934) (end 120.65 106.934) (width 0.6) (layer "B.Cu") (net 2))
 (segment (start 131.891 110.109) (end 129.413 110.109) (width 0.6) (layer "F.Cu") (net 8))
 (segment (start 128.524 110.998) (end 126.9385 110.998) (width 0.6) (layer "F.Cu") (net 8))
 (segment (start 129.413 110.109) (end 128.524 110.998) (width 0.6) (layer "F.Cu") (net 8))
 (via (at 128.524 110.998) (size 0.8) (drill 0.4) (layers "F.Cu" "B.Cu") (free) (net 8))
 (segment (start 128.524 110.998) (end 127 109.474) (width 0.6) (layer "B.Cu") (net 8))
 (segment (start 127 109.474) (end 120.65 109.474) (width 0.6) (layer "B.Cu") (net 8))
 (segment (start 128.524 113.284) (end 128.524 113.03) (width 0.6) (layer "F.Cu") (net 7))
 (segment (start 128.524 113.03) (end 130.175 111.379) (width 0.6) (layer "F.Cu") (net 7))
 (segment (start 128.524 113.284) (end 126.9385 113.284) (width 0.6) (layer "F.Cu") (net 7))
 (segment (start 130.175 111.379) (end 131.891 111.379) (width 0.6) (layer "F.Cu") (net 7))
 (via (at 128.524 113.284) (size 0.8) (drill 0.4) (layers "F.Cu" "B.Cu") (free) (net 7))
 (segment (start 128.524 113.284) (end 127.254 112.014) (width 0.6) (layer "B.Cu") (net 7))
 (segment (start 127.254 112.014) (end 120.65 112.014) (width 0.6) (layer "B.Cu") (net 7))
 (segment (start 128.524 115.062) (end 128.524 115.57) (width 0.6) (layer "F.Cu") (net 9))
 (segment (start 128.524 115.57) (end 126.9385 115.57) (width 0.6) (layer "F.Cu") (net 9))
 (segment (start 130.937 112.649) (end 128.524 115.062) (width 0.6) (layer "F.Cu") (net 9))
 (segment (start 131.891 112.649) (end 130.937 112.649) (width 0.6) (layer "F.Cu") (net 9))
 (via (at 128.524 115.57) (size 0.8) (drill 0.4) (layers "F.Cu" "B.Cu") (free) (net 9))
 (segment (start 127.508 114.554) (end 120.65 114.554) (width 0.6) (layer "B.Cu") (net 9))
 (segment (start 128.524 115.57) (end 127.508 114.554) (width 0.6) (layer "B.Cu") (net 9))
 (segment (start 136.841 111.379) (end 144.8455 111.379) (width 0.6) (layer "F.Cu") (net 3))
 (segment (start 160.528 112.014) (end 160.538 112.024) (width 1) (layer "F.Cu") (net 3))
 (segment (start 160.538 112.024) (end 168.402 112.024) (width 1) (layer "F.Cu") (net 3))
 (segment (start 144.8455 111.379) (end 145.288 111.8215) (width 0.6) (layer "F.Cu") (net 3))
 (segment (start 158.242 113.289) (end 159.517 112.014) (width 1) (layer "F.Cu") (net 3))
 (segment (start 149.9265 113.289) (end 148.844 112.2065) (width 1) (layer "F.Cu") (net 3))
 (segment (start 148.459 111.8215) (end 148.844 112.2065) (width 0.6) (layer "F.Cu") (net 3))
 (segment (start 158.242 113.289) (end 149.9265 113.289) (width 1) (layer "F.Cu") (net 3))
 (segment (start 159.517 112.014) (end 160.528 112.014) (width 1) (layer "F.Cu") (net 3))
 (segment (start 145.288 111.8215) (end 148.459 111.8215) (width 0.6) (layer "F.Cu") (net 3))
 (segment (start 145.288 109.9205) (end 148.205 109.9205) (width 0.6) (layer "F.Cu") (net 5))
 (segment (start 145.0995 110.109) (end 145.288 109.9205) (width 0.6) (layer "F.Cu") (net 5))
 (segment (start 148.205 109.9205) (end 148.844 109.2815) (width 0.6) (layer "F.Cu") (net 5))
 (segment (start 158.242 108.209) (end 149.9165 108.209) (width 1) (layer "F.Cu") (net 5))
 (segment (start 136.841 110.109) (end 145.0995 110.109) (width 0.6) (layer "F.Cu") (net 5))
 (segment (start 149.9165 108.209) (end 148.844 109.2815) (width 1) (layer "F.Cu") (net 5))
 (segment (start 159.517 109.484) (end 168.402 109.484) (width 1) (layer "F.Cu") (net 5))
 (segment (start 158.242 108.209) (end 159.517 109.484) (width 1) (layer "F.Cu") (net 5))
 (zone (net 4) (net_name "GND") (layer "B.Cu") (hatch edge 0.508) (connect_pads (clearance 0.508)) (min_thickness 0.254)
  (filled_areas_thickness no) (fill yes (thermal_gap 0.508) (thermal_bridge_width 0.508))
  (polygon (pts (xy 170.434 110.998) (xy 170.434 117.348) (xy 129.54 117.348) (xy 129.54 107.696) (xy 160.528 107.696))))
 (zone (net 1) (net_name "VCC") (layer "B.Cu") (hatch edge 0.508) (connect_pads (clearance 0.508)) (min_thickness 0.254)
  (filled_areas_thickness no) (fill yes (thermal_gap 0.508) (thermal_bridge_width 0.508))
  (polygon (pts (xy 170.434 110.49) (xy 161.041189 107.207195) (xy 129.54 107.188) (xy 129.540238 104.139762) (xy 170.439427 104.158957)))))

